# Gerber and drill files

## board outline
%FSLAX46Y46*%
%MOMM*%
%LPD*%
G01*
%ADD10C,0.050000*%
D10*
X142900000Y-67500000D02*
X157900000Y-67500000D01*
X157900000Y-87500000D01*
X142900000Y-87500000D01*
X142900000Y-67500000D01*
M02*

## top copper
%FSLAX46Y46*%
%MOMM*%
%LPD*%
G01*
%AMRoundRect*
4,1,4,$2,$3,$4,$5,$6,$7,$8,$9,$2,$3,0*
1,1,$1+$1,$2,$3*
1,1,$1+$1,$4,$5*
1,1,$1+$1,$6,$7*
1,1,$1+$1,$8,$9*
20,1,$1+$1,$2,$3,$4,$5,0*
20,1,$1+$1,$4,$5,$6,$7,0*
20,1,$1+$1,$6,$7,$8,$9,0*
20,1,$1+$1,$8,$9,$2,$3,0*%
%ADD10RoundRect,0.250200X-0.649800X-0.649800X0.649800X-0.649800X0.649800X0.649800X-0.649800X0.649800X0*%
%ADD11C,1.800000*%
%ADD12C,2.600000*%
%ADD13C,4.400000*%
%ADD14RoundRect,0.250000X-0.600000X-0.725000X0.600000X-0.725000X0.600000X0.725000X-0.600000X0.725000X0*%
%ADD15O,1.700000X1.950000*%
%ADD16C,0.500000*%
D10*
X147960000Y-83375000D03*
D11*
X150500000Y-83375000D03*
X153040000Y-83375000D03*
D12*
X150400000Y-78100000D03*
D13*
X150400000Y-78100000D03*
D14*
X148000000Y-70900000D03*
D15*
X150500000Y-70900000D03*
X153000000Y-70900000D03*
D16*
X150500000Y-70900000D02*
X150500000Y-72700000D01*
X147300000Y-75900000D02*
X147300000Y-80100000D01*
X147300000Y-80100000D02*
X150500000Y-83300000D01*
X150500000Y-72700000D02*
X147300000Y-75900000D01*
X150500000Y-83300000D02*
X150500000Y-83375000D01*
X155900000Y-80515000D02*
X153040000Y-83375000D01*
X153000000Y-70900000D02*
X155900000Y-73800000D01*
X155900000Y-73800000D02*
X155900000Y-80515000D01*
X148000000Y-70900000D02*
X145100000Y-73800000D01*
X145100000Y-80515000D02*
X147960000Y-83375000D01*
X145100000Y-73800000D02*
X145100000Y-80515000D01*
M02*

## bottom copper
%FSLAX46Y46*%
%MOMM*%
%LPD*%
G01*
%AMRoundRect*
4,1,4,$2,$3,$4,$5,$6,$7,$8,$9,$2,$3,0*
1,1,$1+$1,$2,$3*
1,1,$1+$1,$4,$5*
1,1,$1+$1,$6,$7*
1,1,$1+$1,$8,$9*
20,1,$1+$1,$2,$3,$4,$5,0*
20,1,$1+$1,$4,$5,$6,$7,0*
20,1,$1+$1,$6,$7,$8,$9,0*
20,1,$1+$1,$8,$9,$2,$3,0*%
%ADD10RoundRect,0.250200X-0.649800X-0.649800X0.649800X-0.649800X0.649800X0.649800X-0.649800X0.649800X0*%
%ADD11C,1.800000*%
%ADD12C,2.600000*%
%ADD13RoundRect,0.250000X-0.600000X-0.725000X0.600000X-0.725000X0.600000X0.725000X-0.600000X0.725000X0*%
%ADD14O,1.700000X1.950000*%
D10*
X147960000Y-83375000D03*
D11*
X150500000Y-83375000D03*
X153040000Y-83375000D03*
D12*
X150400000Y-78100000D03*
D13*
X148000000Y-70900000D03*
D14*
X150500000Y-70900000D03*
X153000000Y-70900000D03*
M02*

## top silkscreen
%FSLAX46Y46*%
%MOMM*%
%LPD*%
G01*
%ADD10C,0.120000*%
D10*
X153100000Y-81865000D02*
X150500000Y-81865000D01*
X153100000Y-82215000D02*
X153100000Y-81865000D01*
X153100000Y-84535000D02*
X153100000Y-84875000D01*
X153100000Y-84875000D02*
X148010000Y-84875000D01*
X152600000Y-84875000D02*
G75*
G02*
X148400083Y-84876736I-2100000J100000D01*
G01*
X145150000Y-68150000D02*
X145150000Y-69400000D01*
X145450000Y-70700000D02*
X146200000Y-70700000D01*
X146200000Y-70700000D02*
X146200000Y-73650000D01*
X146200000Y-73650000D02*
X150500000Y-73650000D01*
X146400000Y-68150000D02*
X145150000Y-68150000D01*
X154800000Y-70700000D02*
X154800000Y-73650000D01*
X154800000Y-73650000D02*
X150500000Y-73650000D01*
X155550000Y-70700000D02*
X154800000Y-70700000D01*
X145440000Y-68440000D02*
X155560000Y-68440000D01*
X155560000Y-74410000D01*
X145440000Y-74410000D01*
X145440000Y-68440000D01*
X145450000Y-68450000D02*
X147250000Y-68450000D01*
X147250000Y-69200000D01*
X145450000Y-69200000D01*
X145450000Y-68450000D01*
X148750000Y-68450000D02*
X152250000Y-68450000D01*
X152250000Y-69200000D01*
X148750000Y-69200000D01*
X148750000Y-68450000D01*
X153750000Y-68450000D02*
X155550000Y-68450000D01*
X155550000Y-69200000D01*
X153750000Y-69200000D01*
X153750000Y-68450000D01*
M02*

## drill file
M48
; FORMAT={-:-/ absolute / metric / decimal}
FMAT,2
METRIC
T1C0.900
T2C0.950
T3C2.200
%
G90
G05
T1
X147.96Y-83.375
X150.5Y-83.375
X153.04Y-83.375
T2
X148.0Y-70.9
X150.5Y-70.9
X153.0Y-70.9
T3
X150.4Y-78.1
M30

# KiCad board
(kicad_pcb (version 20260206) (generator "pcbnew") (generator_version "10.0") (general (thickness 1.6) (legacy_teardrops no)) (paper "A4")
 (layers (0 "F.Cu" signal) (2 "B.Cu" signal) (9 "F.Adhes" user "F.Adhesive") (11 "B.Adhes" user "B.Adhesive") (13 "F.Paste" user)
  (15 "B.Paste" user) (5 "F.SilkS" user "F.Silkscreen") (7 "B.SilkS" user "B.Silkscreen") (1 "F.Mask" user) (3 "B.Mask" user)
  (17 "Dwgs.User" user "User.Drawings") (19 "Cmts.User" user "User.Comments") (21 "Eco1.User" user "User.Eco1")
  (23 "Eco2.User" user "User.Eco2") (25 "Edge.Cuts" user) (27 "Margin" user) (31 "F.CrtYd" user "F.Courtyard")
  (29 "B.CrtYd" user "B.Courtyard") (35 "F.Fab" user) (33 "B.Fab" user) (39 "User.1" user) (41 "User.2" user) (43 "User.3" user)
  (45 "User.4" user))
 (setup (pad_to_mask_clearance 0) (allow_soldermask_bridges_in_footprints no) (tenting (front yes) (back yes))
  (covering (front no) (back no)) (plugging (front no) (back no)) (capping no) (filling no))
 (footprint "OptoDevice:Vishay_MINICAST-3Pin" (layer "F.Cu") (at 147.96 83.375)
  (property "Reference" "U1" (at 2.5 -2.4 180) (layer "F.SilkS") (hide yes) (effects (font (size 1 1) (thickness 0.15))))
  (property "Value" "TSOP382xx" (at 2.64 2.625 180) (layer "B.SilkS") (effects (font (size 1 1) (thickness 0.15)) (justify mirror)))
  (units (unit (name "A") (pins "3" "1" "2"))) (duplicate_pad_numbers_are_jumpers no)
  (fp_line (start 5.14 -1.51) (end 2.54 -1.51) (stroke (width 0.12) (type solid)) (layer "F.SilkS"))
  (fp_line (start 5.14 -1.16) (end 5.14 -1.51) (stroke (width 0.12) (type solid)) (layer "F.SilkS"))
  (fp_line (start 5.14 1.16) (end 5.14 1.5) (stroke (width 0.12) (type solid)) (layer "F.SilkS"))
  (fp_line (start 5.14 1.5) (end 0.05 1.5) (stroke (width 0.12) (type solid)) (layer "F.SilkS"))
  (fp_arc (start 4.64 1.5) (mid 2.540869 3.502379) (end 0.440083 1.501736) (stroke (width 0.12) (type solid)) (layer "F.SilkS"))
  (pad "1" thru_hole roundrect (at 0 0) (size 1.8 1.8) (drill 0.9) (layers "*.Cu" "*.Mask") (remove_unused_layers no)
   (roundrect_rratio 0.139) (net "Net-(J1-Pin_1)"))
  (pad "2" thru_hole circle (at 2.54 0) (size 1.8 1.8) (drill 0.9) (layers "*.Cu" "*.Mask") (remove_unused_layers no) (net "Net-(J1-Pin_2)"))
  (pad "3" thru_hole circle (at 5.08 0) (size 1.8 1.8) (drill 0.9) (layers "*.Cu" "*.Mask") (remove_unused_layers no) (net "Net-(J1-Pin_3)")))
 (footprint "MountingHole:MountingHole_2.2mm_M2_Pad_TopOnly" (layer "F.Cu") (at 150.4 78.1)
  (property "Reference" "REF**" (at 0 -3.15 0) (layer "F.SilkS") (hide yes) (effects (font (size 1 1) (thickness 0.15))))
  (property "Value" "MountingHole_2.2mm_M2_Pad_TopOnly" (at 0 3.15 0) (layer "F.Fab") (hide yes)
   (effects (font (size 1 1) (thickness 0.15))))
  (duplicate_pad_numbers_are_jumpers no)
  (pad "1" thru_hole circle (at 0 0) (size 2.6 2.6) (drill 2.2) (layers "*.Cu" "*.Mask") (remove_unused_layers no) (zone_connect 2))
  (pad "1" connect circle (at 0 0) (size 4.4 4.4) (layers "F.Cu" "F.Mask") (zone_connect 2)))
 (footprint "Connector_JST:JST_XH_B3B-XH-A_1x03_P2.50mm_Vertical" (layer "F.Cu") (at 148 70.9)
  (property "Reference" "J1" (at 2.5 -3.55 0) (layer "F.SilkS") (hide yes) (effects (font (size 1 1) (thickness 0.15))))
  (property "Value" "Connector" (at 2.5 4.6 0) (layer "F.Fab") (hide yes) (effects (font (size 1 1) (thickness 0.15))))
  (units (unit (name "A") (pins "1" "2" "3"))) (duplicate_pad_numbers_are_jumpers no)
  (fp_line (start -2.85 -2.75) (end -2.85 -1.5) (stroke (width 0.12) (type solid)) (layer "F.SilkS"))
  (fp_line (start -2.55 -0.2) (end -1.8 -0.2) (stroke (width 0.12) (type solid)) (layer "F.SilkS"))
  (fp_line (start -1.8 -0.2) (end -1.8 2.75) (stroke (width 0.12) (type solid)) (layer "F.SilkS"))
  (fp_line (start -1.8 2.75) (end 2.5 2.75) (stroke (width 0.12) (type solid)) (layer "F.SilkS"))
  (fp_line (start -1.6 -2.75) (end -2.85 -2.75) (stroke (width 0.12) (type solid)) (layer "F.SilkS"))
  (fp_line (start 6.8 -0.2) (end 6.8 2.75) (stroke (width 0.12) (type solid)) (layer "F.SilkS"))
  (fp_line (start 6.8 2.75) (end 2.5 2.75) (stroke (width 0.12) (type solid)) (layer "F.SilkS"))
  (fp_line (start 7.55 -0.2) (end 6.8 -0.2) (stroke (width 0.12) (type solid)) (layer "F.SilkS"))
  (fp_rect (start -2.56 -2.46) (end 7.56 3.51) (stroke (width 0.12) (type solid)) (fill no) (layer "F.SilkS"))
  (fp_rect (start -2.55 -2.45) (end -0.75 -1.7) (stroke (width 0.12) (type solid)) (fill no) (layer "F.SilkS"))
  (fp_rect (start 0.75 -2.45) (end 4.25 -1.7) (stroke (width 0.12) (type solid)) (fill no) (layer "F.SilkS"))
  (fp_rect (start 5.75 -2.45) (end 7.55 -1.7) (stroke (width 0.12) (type solid)) (fill no) (layer "F.SilkS"))
  (pad "1" thru_hole roundrect (at 0 0) (size 1.7 1.95) (drill 0.95) (layers "*.Cu" "*.Mask") (remove_unused_layers no)
   (roundrect_rratio 0.147059) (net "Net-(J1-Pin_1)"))
  (pad "2" thru_hole oval (at 2.5 0) (size 1.7 1.95) (drill 0.95) (layers "*.Cu" "*.Mask") (remove_unused_layers no) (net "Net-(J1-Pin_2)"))
  (pad "3" thru_hole oval (at 5 0) (size 1.7 1.95) (drill 0.95) (layers "*.Cu" "*.Mask") (remove_unused_layers no) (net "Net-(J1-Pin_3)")))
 (gr_rect (start 142.9 67.5) (end 157.9 87.5) (stroke (width 0.05) (type default)) (fill no) (layer "Edge.Cuts"))
 (segment (start 150.5 70.9) (end 150.5 72.7) (width 0.5) (layer "F.Cu") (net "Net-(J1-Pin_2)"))
 (segment (start 147.3 75.9) (end 147.3 80.1) (width 0.5) (layer "F.Cu") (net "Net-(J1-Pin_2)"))
 (segment (start 147.3 80.1) (end 150.5 83.3) (width 0.5) (layer "F.Cu") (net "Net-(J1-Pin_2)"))
 (segment (start 150.5 72.7) (end 147.3 75.9) (width 0.5) (layer "F.Cu") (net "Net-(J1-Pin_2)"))
 (segment (start 150.5 83.3) (end 150.5 83.375) (width 0.5) (layer "F.Cu") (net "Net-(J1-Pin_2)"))
 (segment (start 155.9 80.515) (end 153.04 83.375) (width 0.5) (layer "F.Cu") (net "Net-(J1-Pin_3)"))
 (segment (start 153 70.9) (end 155.9 73.8) (width 0.5) (layer "F.Cu") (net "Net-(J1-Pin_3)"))
 (segment (start 155.9 73.8) (end 155.9 80.515) (width 0.5) (layer "F.Cu") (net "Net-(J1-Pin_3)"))
 (segment (start 148 70.9) (end 145.1 73.8) (width 0.5) (layer "F.Cu") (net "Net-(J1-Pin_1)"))
 (segment (start 145.1 80.515) (end 147.96 83.375) (width 0.5) (layer "F.Cu") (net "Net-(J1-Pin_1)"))
 (segment (start 145.1 73.8) (end 145.1 80.515) (width 0.5) (layer "F.Cu") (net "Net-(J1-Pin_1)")))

